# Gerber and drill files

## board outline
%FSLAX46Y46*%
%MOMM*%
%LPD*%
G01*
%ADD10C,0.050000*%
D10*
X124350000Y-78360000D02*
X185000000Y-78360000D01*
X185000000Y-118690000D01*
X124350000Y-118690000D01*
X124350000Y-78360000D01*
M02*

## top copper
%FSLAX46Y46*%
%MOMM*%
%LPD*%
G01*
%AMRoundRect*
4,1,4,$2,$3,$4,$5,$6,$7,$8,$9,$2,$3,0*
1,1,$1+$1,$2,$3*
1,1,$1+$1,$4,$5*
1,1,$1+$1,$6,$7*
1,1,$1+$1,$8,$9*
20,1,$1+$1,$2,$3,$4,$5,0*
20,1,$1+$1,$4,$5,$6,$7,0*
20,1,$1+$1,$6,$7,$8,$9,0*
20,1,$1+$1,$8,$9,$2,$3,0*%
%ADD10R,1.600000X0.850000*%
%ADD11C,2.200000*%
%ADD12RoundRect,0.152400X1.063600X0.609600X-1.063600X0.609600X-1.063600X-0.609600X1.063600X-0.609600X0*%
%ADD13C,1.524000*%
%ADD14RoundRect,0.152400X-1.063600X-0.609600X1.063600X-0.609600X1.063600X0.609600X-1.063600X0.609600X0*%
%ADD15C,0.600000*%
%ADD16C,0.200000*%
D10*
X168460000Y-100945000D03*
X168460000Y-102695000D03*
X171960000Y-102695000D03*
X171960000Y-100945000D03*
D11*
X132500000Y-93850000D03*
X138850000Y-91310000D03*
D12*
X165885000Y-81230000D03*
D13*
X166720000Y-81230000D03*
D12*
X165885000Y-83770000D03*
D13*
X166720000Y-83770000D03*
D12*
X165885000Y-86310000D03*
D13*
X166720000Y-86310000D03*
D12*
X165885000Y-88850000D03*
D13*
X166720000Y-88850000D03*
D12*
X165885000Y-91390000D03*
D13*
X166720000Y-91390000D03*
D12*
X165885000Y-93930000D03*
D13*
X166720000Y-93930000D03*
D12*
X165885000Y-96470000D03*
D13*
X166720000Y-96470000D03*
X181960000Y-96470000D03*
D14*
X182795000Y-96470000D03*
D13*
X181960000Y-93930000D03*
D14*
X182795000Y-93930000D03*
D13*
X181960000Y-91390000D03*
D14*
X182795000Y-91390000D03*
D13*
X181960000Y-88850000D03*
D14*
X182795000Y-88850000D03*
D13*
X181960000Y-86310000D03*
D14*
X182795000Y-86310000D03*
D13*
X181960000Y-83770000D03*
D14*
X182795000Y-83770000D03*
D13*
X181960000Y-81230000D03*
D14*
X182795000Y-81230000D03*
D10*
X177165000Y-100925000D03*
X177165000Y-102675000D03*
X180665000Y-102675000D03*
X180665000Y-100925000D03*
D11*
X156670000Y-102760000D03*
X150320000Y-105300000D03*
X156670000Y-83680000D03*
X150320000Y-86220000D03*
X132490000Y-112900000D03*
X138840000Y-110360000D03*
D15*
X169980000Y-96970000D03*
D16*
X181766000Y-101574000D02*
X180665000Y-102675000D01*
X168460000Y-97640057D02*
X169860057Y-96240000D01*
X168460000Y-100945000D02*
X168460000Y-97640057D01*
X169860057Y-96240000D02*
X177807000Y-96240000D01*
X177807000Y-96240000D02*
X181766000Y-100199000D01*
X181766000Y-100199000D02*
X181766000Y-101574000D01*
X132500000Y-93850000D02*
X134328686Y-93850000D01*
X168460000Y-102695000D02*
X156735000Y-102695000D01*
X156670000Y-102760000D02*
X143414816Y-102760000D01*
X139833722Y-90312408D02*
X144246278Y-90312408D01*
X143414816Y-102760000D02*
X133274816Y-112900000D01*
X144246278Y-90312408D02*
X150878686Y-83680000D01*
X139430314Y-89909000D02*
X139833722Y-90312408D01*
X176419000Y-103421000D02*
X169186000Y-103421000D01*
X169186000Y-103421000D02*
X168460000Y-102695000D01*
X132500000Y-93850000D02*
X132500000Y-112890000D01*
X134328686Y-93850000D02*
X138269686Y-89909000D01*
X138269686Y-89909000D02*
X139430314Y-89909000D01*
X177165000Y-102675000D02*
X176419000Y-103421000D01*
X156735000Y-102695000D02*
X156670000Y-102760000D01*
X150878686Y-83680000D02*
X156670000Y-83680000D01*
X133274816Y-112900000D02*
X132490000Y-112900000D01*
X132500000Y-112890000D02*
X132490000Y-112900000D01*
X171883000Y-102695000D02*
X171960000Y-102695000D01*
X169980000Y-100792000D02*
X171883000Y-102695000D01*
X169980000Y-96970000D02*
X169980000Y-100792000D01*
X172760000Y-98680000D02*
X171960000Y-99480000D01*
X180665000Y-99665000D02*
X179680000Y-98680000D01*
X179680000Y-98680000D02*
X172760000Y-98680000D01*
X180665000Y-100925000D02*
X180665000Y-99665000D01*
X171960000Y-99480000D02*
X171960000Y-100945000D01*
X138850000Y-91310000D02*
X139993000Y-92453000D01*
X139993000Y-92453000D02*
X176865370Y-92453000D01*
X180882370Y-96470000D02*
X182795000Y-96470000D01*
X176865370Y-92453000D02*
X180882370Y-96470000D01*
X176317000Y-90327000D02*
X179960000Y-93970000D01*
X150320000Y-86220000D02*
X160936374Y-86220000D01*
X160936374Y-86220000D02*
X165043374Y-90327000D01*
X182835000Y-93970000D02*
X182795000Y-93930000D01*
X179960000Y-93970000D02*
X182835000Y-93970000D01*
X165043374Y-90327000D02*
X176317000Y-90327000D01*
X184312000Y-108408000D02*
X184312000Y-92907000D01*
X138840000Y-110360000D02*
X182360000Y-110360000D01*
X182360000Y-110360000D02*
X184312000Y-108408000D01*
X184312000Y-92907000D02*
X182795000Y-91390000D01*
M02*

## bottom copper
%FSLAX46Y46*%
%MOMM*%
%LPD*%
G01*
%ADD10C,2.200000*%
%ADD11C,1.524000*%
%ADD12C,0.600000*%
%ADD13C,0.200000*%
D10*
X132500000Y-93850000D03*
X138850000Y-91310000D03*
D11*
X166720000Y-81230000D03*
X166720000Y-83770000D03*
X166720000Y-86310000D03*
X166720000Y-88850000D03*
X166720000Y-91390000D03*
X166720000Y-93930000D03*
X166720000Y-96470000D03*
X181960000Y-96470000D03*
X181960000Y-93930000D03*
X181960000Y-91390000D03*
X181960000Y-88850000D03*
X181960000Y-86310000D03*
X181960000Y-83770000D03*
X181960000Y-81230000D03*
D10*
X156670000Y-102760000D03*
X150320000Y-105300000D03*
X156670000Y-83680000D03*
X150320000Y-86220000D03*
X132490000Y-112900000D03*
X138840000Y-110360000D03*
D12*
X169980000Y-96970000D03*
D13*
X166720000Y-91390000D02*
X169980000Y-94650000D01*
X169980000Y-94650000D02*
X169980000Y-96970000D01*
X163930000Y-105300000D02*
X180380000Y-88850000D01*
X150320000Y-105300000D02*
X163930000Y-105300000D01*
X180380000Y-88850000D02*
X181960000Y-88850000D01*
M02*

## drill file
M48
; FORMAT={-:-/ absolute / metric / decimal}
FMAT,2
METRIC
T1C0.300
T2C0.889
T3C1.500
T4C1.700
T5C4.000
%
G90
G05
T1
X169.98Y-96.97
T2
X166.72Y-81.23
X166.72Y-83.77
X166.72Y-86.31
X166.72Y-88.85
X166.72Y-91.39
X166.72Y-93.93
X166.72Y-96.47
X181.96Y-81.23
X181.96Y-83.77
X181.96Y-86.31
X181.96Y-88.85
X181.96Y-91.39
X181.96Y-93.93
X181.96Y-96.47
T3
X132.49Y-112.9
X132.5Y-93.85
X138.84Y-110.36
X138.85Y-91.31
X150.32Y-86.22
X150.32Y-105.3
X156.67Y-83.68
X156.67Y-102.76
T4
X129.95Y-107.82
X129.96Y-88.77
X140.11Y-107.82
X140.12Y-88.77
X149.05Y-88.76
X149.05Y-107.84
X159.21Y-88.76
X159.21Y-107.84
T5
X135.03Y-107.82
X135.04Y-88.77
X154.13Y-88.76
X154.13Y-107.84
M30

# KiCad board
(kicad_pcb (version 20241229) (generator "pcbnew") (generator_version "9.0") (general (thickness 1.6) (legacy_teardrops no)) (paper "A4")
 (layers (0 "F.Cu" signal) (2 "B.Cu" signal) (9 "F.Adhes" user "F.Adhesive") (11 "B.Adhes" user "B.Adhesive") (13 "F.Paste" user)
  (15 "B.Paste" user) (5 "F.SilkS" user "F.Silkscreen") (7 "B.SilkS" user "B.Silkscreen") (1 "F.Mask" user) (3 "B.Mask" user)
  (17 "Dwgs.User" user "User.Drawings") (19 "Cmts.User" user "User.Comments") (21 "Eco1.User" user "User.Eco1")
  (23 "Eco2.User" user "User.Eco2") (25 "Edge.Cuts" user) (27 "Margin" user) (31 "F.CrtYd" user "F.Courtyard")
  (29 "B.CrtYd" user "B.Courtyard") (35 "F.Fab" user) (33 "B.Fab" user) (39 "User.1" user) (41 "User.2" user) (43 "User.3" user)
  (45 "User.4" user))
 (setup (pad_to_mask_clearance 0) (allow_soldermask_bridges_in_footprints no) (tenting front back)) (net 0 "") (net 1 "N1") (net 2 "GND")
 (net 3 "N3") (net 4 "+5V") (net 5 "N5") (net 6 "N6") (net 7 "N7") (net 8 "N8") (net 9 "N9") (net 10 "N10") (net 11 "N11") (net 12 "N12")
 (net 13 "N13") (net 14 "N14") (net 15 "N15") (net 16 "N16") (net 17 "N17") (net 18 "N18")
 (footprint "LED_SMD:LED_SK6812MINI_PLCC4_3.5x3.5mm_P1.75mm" (layer "F.Cu") (at 170.21 101.82)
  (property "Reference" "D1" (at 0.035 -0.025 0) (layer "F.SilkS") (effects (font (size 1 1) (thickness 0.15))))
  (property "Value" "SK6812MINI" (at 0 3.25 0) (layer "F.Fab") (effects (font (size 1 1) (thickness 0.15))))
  (pad "1" smd rect (at -1.75 -0.875) (size 1.6 0.85) (layers "F.Cu" "F.Mask" "F.Paste") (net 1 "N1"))
  (pad "2" smd rect (at -1.75 0.875) (size 1.6 0.85) (layers "F.Cu" "F.Mask" "F.Paste") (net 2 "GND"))
  (pad "3" smd rect (at 1.75 0.875) (size 1.6 0.85) (layers "F.Cu" "F.Mask" "F.Paste") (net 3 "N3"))
  (pad "4" smd rect (at 1.75 -0.875) (size 1.6 0.85) (layers "F.Cu" "F.Mask" "F.Paste") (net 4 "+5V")))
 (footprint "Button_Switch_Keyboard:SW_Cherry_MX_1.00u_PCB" (layer "F.Cu") (at 132.5 93.85 180)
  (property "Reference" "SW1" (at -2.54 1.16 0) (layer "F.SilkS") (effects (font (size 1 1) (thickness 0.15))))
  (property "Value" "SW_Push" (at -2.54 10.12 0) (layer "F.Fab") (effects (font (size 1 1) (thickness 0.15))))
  (pad "" np_thru_hole circle (at -7.62 5.08 180) (size 1.7 1.7) (drill 1.7) (layers "*.Cu" "*.Mask"))
  (pad "" np_thru_hole circle (at -2.54 5.08 180) (size 4 4) (drill 4) (layers "*.Cu" "*.Mask"))
  (pad "" np_thru_hole circle (at 2.54 5.08 180) (size 1.7 1.7) (drill 1.7) (layers "*.Cu" "*.Mask"))
  (pad "1" thru_hole circle (at 0 0 180) (size 2.2 2.2) (drill 1.5) (layers "*.Cu" "*.Mask") (remove_unused_layers no) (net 2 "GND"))
  (pad "2" thru_hole circle (at -6.35 2.54 180) (size 2.2 2.2) (drill 1.5) (layers "*.Cu" "*.Mask") (remove_unused_layers no) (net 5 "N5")))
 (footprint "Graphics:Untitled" (layer "F.Cu") (at 174.42 109.89 90)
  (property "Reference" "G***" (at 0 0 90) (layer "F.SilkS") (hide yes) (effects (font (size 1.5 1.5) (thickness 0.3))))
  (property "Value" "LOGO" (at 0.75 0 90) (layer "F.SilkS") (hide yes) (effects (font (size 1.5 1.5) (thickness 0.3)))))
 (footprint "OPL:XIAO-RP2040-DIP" (layer "F.Cu") (at 174.34 88.85)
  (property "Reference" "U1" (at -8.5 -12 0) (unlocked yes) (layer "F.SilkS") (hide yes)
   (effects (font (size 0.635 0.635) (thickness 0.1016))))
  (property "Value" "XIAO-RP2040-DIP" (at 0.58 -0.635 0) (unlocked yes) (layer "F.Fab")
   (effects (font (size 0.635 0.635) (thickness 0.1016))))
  (pad "1" smd roundrect (at -8.455 -7.62 180) (size 2.432 1.524) (layers "F.Cu" "F.Mask") (roundrect_rratio 0.1) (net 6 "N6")
   (thermal_bridge_angle 45))
  (pad "1" thru_hole circle (at -7.62 -7.62 180) (size 1.524 1.524) (drill 0.889) (layers "*.Cu" "*.Mask") (remove_unused_layers no)
   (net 6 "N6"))
  (pad "2" smd roundrect (at -8.455 -5.08 180) (size 2.432 1.524) (layers "F.Cu" "F.Mask") (roundrect_rratio 0.1) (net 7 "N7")
   (thermal_bridge_angle 45))
  (pad "2" thru_hole circle (at -7.62 -5.08 180) (size 1.524 1.524) (drill 0.889) (layers "*.Cu" "*.Mask") (remove_unused_layers no)
   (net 7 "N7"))
  (pad "3" smd roundrect (at -8.455 -2.54 180) (size 2.432 1.524) (layers "F.Cu" "F.Mask") (roundrect_rratio 0.1) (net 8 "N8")
   (thermal_bridge_angle 45))
  (pad "3" thru_hole circle (at -7.62 -2.54 180) (size 1.524 1.524) (drill 0.889) (layers "*.Cu" "*.Mask") (remove_unused_layers no)
   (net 8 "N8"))
  (pad "4" smd roundrect (at -8.455 0 180) (size 2.432 1.524) (layers "F.Cu" "F.Mask") (roundrect_rratio 0.1) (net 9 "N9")
   (thermal_bridge_angle 45))
  (pad "4" thru_hole circle (at -7.62 0 180) (size 1.524 1.524) (drill 0.889) (layers "*.Cu" "*.Mask") (remove_unused_layers no)
   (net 9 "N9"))
  (pad "5" smd roundrect (at -8.455 2.54 180) (size 2.432 1.524) (layers "F.Cu" "F.Mask") (roundrect_rratio 0.1) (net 3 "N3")
   (thermal_bridge_angle 45))
  (pad "5" thru_hole circle (at -7.62 2.54 180) (size 1.524 1.524) (drill 0.889) (layers "*.Cu" "*.Mask") (remove_unused_layers no)
   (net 3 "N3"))
  (pad "6" smd roundrect (at -8.455 5.08 180) (size 2.432 1.524) (layers "F.Cu" "F.Mask") (roundrect_rratio 0.1) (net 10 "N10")
   (thermal_bridge_angle 45))
  (pad "6" thru_hole circle (at -7.62 5.08 180) (size 1.524 1.524) (drill 0.889) (layers "*.Cu" "*.Mask") (remove_unused_layers no)
   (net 10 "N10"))
  (pad "7" smd roundrect (at -8.455 7.62 180) (size 2.432 1.524) (layers "F.Cu" "F.Mask") (roundrect_rratio 0.1) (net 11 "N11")
   (thermal_bridge_angle 45))
  (pad "7" thru_hole circle (at -7.62 7.62 180) (size 1.524 1.524) (drill 0.889) (layers "*.Cu" "*.Mask") (remove_unused_layers no)
   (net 11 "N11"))
  (pad "8" thru_hole circle (at 7.62 7.62) (size 1.524 1.524) (drill 0.889) (layers "*.Cu" "*.Mask") (remove_unused_layers no) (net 5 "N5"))
  (pad "8" smd roundrect (at 8.455 7.62) (size 2.432 1.524) (layers "F.Cu" "F.Mask") (roundrect_rratio 0.1) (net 5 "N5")
   (thermal_bridge_angle 45))
  (pad "9" thru_hole circle (at 7.62 5.08) (size 1.524 1.524) (drill 0.889) (layers "*.Cu" "*.Mask") (remove_unused_layers no)
   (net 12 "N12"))
  (pad "9" smd roundrect (at 8.455 5.08) (size 2.432 1.524) (layers "F.Cu" "F.Mask") (roundrect_rratio 0.1) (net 12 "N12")
   (thermal_bridge_angle 45))
  (pad "10" thru_hole circle (at 7.62 2.54) (size 1.524 1.524) (drill 0.889) (layers "*.Cu" "*.Mask") (remove_unused_layers no)
   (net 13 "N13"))
  (pad "10" smd roundrect (at 8.455 2.54) (size 2.432 1.524) (layers "F.Cu" "F.Mask") (roundrect_rratio 0.1) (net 13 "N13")
   (thermal_bridge_angle 45))
  (pad "11" thru_hole circle (at 7.62 0) (size 1.524 1.524) (drill 0.889) (layers "*.Cu" "*.Mask") (remove_unused_layers no) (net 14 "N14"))
  (pad "11" smd roundrect (at 8.455 0) (size 2.432 1.524) (layers "F.Cu" "F.Mask") (roundrect_rratio 0.1) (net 14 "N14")
   (thermal_bridge_angle 45))
  (pad "12" thru_hole circle (at 7.62 -2.54) (size 1.524 1.524) (drill 0.889) (layers "*.Cu" "*.Mask") (remove_unused_layers no)
   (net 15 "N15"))
  (pad "12" smd roundrect (at 8.455 -2.54) (size 2.432 1.524) (layers "F.Cu" "F.Mask") (roundrect_rratio 0.1) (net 15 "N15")
   (thermal_bridge_angle 45))
  (pad "13" thru_hole circle (at 7.62 -5.08) (size 1.524 1.524) (drill 0.889) (layers "*.Cu" "*.Mask") (remove_unused_layers no)
   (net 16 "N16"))
  (pad "13" smd roundrect (at 8.455 -5.08) (size 2.432 1.524) (layers "F.Cu" "F.Mask") (roundrect_rratio 0.1) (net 16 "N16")
   (thermal_bridge_angle 45))
  (pad "14" thru_hole circle (at 7.62 -7.62) (size 1.524 1.524) (drill 0.889) (layers "*.Cu" "*.Mask") (remove_unused_layers no)
   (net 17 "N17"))
  (pad "14" smd roundrect (at 8.455 -7.62) (size 2.432 1.524) (layers "F.Cu" "F.Mask") (roundrect_rratio 0.1) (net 17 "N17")
   (thermal_bridge_angle 45)))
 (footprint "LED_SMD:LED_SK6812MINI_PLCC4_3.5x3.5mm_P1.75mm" (layer "F.Cu") (at 178.915 101.8)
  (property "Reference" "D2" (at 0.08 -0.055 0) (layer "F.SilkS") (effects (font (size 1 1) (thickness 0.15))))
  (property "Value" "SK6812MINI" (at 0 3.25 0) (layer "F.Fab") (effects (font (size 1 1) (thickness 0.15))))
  (pad "1" smd rect (at -1.75 -0.875) (size 1.6 0.85) (layers "F.Cu" "F.Mask" "F.Paste") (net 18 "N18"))
  (pad "2" smd rect (at -1.75 0.875) (size 1.6 0.85) (layers "F.Cu" "F.Mask" "F.Paste") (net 2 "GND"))
  (pad "3" smd rect (at 1.75 0.875) (size 1.6 0.85) (layers "F.Cu" "F.Mask" "F.Paste") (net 1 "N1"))
  (pad "4" smd rect (at 1.75 -0.875) (size 1.6 0.85) (layers "F.Cu" "F.Mask" "F.Paste") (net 4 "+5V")))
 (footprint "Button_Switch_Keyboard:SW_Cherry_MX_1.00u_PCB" (layer "F.Cu") (at 156.67 102.76)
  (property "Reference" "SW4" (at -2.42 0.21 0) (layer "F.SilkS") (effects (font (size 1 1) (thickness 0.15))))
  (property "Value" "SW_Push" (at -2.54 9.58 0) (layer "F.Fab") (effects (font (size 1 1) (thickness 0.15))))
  (pad "" np_thru_hole circle (at -7.62 5.08) (size 1.7 1.7) (drill 1.7) (layers "*.Cu" "*.Mask"))
  (pad "" np_thru_hole circle (at -2.54 5.08) (size 4 4) (drill 4) (layers "*.Cu" "*.Mask"))
  (pad "" np_thru_hole circle (at 2.54 5.08) (size 1.7 1.7) (drill 1.7) (layers "*.Cu" "*.Mask"))
  (pad "1" thru_hole circle (at 0 0) (size 2.2 2.2) (drill 1.5) (layers "*.Cu" "*.Mask") (remove_unused_layers no) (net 2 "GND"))
  (pad "2" thru_hole circle (at -6.35 2.54) (size 2.2 2.2) (drill 1.5) (layers "*.Cu" "*.Mask") (remove_unused_layers no) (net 14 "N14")))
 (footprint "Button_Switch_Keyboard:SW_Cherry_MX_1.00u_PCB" (layer "F.Cu") (at 156.67 83.68)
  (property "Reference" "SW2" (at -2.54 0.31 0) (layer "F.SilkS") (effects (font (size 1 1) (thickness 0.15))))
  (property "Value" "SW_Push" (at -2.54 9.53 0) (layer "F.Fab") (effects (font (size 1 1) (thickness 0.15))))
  (pad "" np_thru_hole circle (at -7.62 5.08) (size 1.7 1.7) (drill 1.7) (layers "*.Cu" "*.Mask"))
  (pad "" np_thru_hole circle (at -2.54 5.08) (size 4 4) (drill 4) (layers "*.Cu" "*.Mask"))
  (pad "" np_thru_hole circle (at 2.54 5.08) (size 1.7 1.7) (drill 1.7) (layers "*.Cu" "*.Mask"))
  (pad "1" thru_hole circle (at 0 0) (size 2.2 2.2) (drill 1.5) (layers "*.Cu" "*.Mask") (remove_unused_layers no) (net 2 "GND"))
  (pad "2" thru_hole circle (at -6.35 2.54) (size 2.2 2.2) (drill 1.5) (layers "*.Cu" "*.Mask") (remove_unused_layers no) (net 12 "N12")))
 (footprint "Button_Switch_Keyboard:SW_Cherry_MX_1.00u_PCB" (layer "F.Cu") (at 132.49 112.9 180)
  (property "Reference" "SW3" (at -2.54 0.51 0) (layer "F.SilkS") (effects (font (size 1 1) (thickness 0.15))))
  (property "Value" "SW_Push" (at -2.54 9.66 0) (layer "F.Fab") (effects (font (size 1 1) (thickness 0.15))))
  (pad "" np_thru_hole circle (at -7.62 5.08 180) (size 1.7 1.7) (drill 1.7) (layers "*.Cu" "*.Mask"))
  (pad "" np_thru_hole circle (at -2.54 5.08 180) (size 4 4) (drill 4) (layers "*.Cu" "*.Mask"))
  (pad "" np_thru_hole circle (at 2.54 5.08 180) (size 1.7 1.7) (drill 1.7) (layers "*.Cu" "*.Mask"))
  (pad "1" thru_hole circle (at 0 0 180) (size 2.2 2.2) (drill 1.5) (layers "*.Cu" "*.Mask") (remove_unused_layers no) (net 2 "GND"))
  (pad "2" thru_hole circle (at -6.35 2.54 180) (size 2.2 2.2) (drill 1.5) (layers "*.Cu" "*.Mask") (remove_unused_layers no) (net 13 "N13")))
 (gr_rect (start 124.35 78.36) (end 185 118.69) (stroke (width 0.05) (type default)) (fill no) (layer "Edge.Cuts"))
 (segment (start 181.766 101.574) (end 180.665 102.675) (width 0.2) (layer "F.Cu") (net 1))
 (segment (start 168.46 97.640057) (end 169.860057 96.24) (width 0.2) (layer "F.Cu") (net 1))
 (segment (start 168.46 100.945) (end 168.46 97.640057) (width 0.2) (layer "F.Cu") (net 1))
 (segment (start 169.860057 96.24) (end 177.807 96.24) (width 0.2) (layer "F.Cu") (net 1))
 (segment (start 177.807 96.24) (end 181.766 100.199) (width 0.2) (layer "F.Cu") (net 1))
 (segment (start 181.766 100.199) (end 181.766 101.574) (width 0.2) (layer "F.Cu") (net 1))
 (segment (start 132.5 93.85) (end 134.328686 93.85) (width 0.2) (layer "F.Cu") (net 2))
 (segment (start 168.46 102.695) (end 156.735 102.695) (width 0.2) (layer "F.Cu") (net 2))
 (segment (start 156.67 102.76) (end 143.414816 102.76) (width 0.2) (layer "F.Cu") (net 2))
 (segment (start 139.833722 90.312408) (end 144.246278 90.312408) (width 0.2) (layer "F.Cu") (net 2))
 (segment (start 143.414816 102.76) (end 133.274816 112.9) (width 0.2) (layer "F.Cu") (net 2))
 (segment (start 144.246278 90.312408) (end 150.878686 83.68) (width 0.2) (layer "F.Cu") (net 2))
 (segment (start 139.430314 89.909) (end 139.833722 90.312408) (width 0.2) (layer "F.Cu") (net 2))
 (segment (start 176.419 103.421) (end 169.186 103.421) (width 0.2) (layer "F.Cu") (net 2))
 (segment (start 169.186 103.421) (end 168.46 102.695) (width 0.2) (layer "F.Cu") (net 2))
 (segment (start 132.5 93.85) (end 132.5 112.89) (width 0.2) (layer "F.Cu") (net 2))
 (segment (start 134.328686 93.85) (end 138.269686 89.909) (width 0.2) (layer "F.Cu") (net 2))
 (segment (start 138.269686 89.909) (end 139.430314 89.909) (width 0.2) (layer "F.Cu") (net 2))
 (segment (start 177.165 102.675) (end 176.419 103.421) (width 0.2) (layer "F.Cu") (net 2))
 (segment (start 156.735 102.695) (end 156.67 102.76) (width 0.2) (layer "F.Cu") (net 2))
 (segment (start 150.878686 83.68) (end 156.67 83.68) (width 0.2) (layer "F.Cu") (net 2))
 (segment (start 133.274816 112.9) (end 132.49 112.9) (width 0.2) (layer "F.Cu") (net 2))
 (segment (start 132.5 112.89) (end 132.49 112.9) (width 0.2) (layer "F.Cu") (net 2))
 (segment (start 171.883 102.695) (end 171.96 102.695) (width 0.2) (layer "F.Cu") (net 3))
 (segment (start 169.98 100.792) (end 171.883 102.695) (width 0.2) (layer "F.Cu") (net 3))
 (segment (start 169.98 96.97) (end 169.98 100.792) (width 0.2) (layer "F.Cu") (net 3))
 (via (at 169.98 96.97) (size 0.6) (drill 0.3) (layers "F.Cu" "B.Cu") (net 3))
 (segment (start 166.72 91.39) (end 169.98 94.65) (width 0.2) (layer "B.Cu") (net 3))
 (segment (start 169.98 94.65) (end 169.98 96.97) (width 0.2) (layer "B.Cu") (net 3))
 (segment (start 172.76 98.68) (end 171.96 99.48) (width 0.2) (layer "F.Cu") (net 4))
 (segment (start 180.665 99.665) (end 179.68 98.68) (width 0.2) (layer "F.Cu") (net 4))
 (segment (start 179.68 98.68) (end 172.76 98.68) (width 0.2) (layer "F.Cu") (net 4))
 (segment (start 180.665 100.925) (end 180.665 99.665) (width 0.2) (layer "F.Cu") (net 4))
 (segment (start 171.96 99.48) (end 171.96 100.945) (width 0.2) (layer "F.Cu") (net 4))
 (segment (start 138.85 91.31) (end 139.993 92.453) (width 0.2) (layer "F.Cu") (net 5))
 (segment (start 139.993 92.453) (end 176.86537 92.453) (width 0.2) (layer "F.Cu") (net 5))
 (segment (start 180.88237 96.47) (end 182.795 96.47) (width 0.2) (layer "F.Cu") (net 5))
 (segment (start 176.86537 92.453) (end 180.88237 96.47) (width 0.2) (layer "F.Cu") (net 5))
 (segment (start 176.317 90.327) (end 179.96 93.97) (width 0.2) (layer "F.Cu") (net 12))
 (segment (start 150.32 86.22) (end 160.936374 86.22) (width 0.2) (layer "F.Cu") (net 12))
 (segment (start 160.936374 86.22) (end 165.043374 90.327) (width 0.2) (layer "F.Cu") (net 12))
 (segment (start 182.835 93.97) (end 182.795 93.93) (width 0.2) (layer "F.Cu") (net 12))
 (segment (start 179.96 93.97) (end 182.835 93.97) (width 0.2) (layer "F.Cu") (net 12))
 (segment (start 165.043374 90.327) (end 176.317 90.327) (width 0.2) (layer "F.Cu") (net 12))
 (segment (start 184.312 108.408) (end 184.312 92.907) (width 0.2) (layer "F.Cu") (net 13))
 (segment (start 138.84 110.36) (end 182.36 110.36) (width 0.2) (layer "F.Cu") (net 13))
 (segment (start 182.36 110.36) (end 184.312 108.408) (width 0.2) (layer "F.Cu") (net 13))
 (segment (start 184.312 92.907) (end 182.795 91.39) (width 0.2) (layer "F.Cu") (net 13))
 (segment (start 163.93 105.3) (end 180.38 88.85) (width 0.2) (layer "B.Cu") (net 14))
 (segment (start 150.32 105.3) (end 163.93 105.3) (width 0.2) (layer "B.Cu") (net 14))
 (segment (start 180.38 88.85) (end 181.96 88.85) (width 0.2) (layer "B.Cu") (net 14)))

